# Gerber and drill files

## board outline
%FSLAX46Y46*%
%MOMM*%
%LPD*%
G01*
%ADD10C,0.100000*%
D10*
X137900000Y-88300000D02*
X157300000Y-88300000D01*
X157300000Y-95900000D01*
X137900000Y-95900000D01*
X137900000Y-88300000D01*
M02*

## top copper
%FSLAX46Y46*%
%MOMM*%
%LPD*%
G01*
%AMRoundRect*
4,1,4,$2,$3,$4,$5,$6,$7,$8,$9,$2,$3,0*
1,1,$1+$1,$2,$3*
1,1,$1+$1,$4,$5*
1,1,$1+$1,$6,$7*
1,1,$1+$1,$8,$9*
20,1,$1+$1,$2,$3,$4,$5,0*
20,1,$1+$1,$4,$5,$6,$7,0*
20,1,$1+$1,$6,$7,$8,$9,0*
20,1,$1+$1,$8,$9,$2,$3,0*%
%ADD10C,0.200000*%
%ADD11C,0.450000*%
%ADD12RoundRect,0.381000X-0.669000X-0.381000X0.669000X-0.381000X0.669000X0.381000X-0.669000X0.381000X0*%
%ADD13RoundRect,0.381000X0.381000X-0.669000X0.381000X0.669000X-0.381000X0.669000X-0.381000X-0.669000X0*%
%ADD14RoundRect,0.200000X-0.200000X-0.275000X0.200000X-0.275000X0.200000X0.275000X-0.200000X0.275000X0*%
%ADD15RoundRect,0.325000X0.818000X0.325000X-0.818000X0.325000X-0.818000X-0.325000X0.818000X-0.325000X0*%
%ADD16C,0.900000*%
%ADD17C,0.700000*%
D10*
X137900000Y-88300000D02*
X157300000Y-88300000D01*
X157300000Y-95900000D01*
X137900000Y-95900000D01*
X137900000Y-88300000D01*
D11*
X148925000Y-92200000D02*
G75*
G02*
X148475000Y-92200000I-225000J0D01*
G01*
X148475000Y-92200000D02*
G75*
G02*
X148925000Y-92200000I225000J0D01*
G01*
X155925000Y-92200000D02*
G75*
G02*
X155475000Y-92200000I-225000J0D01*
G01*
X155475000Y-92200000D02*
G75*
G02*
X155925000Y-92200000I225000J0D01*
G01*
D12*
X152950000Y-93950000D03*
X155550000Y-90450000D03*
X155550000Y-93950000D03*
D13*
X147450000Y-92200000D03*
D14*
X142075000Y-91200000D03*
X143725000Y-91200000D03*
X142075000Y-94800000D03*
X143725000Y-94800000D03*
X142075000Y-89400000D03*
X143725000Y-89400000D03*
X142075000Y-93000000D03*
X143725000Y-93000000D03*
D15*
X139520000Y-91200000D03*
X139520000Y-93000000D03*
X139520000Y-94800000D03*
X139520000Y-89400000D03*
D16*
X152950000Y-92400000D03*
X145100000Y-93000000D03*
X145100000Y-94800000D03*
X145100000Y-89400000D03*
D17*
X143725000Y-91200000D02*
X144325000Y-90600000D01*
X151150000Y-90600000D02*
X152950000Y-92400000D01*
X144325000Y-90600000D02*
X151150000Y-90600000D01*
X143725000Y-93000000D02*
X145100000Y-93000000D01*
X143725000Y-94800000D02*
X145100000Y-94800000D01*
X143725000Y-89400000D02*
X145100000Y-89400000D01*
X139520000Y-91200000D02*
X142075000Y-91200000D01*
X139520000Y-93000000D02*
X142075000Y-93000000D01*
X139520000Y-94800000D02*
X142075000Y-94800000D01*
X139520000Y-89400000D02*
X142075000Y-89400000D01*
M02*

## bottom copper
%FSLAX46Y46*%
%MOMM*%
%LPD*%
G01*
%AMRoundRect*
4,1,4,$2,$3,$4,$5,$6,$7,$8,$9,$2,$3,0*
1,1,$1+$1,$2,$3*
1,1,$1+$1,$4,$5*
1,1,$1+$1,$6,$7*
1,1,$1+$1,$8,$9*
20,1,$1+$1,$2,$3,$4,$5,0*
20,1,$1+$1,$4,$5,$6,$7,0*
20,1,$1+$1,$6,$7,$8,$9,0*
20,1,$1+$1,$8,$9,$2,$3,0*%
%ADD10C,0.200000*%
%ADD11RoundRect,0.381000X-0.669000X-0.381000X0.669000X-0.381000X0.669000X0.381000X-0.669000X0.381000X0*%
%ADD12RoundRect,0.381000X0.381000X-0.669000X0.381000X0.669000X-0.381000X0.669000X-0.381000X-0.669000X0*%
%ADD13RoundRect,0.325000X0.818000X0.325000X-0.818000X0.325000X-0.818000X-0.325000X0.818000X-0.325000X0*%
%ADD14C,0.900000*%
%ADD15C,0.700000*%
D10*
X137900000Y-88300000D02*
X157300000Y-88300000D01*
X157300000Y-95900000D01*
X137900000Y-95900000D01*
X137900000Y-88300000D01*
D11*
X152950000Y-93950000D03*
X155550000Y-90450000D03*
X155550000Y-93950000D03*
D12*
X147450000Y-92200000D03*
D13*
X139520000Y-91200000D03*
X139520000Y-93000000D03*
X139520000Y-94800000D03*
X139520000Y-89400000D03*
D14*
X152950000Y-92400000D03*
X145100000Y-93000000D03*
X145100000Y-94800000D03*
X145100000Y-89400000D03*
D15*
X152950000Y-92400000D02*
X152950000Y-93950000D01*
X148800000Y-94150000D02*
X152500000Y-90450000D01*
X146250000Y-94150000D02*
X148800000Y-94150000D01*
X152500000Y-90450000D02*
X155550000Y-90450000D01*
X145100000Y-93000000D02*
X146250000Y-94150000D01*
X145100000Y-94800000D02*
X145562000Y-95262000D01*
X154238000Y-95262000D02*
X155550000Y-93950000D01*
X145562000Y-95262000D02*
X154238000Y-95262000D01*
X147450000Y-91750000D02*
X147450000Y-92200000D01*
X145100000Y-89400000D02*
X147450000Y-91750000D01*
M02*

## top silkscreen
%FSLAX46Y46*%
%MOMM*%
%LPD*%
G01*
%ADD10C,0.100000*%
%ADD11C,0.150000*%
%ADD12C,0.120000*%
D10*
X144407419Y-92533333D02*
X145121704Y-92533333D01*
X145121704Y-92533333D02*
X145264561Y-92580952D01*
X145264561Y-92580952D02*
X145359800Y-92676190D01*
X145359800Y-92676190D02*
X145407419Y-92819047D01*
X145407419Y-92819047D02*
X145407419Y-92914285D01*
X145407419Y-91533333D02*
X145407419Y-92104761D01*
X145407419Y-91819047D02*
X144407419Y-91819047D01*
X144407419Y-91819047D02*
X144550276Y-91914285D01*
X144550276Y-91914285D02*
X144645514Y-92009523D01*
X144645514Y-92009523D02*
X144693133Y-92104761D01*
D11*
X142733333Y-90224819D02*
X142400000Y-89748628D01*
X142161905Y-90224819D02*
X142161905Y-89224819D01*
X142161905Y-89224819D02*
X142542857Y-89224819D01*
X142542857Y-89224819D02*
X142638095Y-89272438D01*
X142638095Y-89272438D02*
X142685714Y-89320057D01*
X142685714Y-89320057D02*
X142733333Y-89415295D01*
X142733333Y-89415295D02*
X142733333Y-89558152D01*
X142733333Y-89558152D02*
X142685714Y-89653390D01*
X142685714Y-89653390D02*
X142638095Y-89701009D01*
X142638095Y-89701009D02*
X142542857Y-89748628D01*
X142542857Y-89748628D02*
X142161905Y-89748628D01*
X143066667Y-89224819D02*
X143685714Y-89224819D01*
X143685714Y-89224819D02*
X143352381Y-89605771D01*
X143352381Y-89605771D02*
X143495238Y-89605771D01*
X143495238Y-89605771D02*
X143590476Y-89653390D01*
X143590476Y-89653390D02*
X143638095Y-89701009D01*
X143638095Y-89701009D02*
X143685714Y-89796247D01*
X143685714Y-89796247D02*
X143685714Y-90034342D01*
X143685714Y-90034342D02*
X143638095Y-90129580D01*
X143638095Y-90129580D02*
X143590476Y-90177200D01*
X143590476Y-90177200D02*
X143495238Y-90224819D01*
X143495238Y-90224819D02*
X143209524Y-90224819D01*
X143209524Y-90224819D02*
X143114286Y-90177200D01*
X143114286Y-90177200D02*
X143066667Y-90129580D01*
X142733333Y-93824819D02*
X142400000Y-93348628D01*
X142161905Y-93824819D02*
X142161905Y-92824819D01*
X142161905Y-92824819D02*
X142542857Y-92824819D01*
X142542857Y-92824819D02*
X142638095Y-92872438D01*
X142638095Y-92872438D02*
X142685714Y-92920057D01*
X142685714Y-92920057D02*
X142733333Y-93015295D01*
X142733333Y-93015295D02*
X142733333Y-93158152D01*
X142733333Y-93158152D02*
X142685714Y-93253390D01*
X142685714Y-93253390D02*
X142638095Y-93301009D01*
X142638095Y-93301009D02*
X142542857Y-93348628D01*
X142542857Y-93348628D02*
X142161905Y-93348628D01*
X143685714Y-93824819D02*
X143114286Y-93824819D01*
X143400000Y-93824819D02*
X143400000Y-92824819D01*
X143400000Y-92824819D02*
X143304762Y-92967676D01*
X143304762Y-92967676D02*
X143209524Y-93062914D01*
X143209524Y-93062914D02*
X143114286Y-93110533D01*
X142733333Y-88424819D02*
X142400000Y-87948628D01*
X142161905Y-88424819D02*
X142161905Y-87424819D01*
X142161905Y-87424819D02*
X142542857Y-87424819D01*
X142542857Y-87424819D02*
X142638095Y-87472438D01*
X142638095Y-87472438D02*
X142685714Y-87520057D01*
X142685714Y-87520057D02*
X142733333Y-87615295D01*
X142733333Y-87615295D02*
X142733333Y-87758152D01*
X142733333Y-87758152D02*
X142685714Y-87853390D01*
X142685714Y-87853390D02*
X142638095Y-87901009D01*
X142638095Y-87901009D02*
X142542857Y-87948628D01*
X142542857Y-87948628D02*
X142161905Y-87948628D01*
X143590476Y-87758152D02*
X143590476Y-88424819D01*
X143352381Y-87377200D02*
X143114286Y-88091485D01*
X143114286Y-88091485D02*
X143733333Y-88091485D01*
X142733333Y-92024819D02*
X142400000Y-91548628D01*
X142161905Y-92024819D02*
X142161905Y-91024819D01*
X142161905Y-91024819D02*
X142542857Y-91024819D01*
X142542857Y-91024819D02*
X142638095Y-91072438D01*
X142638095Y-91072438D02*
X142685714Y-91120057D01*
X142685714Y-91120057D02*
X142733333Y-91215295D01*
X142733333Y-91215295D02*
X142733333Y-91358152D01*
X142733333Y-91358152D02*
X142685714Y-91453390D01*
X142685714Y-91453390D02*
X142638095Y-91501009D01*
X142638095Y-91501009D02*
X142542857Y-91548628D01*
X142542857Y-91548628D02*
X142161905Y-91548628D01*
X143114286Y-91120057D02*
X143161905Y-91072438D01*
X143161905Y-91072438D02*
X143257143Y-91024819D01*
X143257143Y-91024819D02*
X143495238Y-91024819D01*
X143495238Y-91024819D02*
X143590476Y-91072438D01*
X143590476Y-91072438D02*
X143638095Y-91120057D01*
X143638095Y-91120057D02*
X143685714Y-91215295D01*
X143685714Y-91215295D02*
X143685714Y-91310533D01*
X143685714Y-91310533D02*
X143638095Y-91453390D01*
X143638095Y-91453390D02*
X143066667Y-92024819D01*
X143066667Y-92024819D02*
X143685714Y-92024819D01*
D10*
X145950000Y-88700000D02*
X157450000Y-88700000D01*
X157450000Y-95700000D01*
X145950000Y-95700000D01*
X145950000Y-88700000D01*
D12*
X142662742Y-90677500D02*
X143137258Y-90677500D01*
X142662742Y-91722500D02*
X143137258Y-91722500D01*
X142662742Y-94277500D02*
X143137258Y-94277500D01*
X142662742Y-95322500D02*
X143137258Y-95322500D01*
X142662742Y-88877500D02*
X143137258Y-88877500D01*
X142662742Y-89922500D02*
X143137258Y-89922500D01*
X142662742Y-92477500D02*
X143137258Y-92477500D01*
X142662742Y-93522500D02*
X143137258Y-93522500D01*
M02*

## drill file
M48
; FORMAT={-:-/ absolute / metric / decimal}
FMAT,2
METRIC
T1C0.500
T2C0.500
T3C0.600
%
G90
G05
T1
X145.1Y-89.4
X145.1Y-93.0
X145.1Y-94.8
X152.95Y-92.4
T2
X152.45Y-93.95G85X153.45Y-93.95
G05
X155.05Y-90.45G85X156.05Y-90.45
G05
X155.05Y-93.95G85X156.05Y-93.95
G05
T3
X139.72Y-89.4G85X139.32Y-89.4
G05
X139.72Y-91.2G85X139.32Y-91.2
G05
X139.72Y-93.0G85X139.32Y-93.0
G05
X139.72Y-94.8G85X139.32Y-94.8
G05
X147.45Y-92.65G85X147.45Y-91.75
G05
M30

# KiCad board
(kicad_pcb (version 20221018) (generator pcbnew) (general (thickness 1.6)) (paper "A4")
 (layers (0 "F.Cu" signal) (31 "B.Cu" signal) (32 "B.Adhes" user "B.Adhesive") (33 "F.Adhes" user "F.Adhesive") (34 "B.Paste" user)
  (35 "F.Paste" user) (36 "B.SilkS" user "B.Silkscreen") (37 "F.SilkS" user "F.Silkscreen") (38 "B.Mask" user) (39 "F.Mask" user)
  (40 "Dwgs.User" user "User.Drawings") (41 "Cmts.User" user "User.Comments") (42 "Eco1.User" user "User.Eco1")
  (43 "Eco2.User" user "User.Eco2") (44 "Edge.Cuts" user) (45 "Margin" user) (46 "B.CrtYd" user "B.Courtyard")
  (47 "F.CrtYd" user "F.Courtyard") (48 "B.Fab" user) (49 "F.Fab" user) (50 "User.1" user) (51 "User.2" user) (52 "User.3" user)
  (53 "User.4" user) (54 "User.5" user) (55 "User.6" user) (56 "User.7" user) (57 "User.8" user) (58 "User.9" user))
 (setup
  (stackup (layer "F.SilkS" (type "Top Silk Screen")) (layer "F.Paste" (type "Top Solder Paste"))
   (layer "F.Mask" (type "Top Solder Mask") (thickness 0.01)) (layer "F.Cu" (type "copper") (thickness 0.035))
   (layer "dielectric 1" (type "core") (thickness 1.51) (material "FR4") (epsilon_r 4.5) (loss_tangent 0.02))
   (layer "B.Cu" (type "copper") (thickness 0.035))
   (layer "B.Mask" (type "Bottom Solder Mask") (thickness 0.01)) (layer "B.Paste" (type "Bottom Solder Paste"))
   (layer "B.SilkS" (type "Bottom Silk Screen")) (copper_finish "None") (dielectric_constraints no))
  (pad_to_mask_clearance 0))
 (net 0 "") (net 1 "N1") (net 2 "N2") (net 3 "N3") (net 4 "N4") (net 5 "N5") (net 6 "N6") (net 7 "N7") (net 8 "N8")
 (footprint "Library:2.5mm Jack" (layer "F.Cu") (at 157.45 92.2 90)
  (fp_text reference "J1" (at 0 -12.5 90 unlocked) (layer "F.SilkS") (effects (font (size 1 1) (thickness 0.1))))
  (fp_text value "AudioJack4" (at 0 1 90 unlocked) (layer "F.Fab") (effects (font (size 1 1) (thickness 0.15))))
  (fp_circle (center 0 -8.75) (end 0.4 -8.75) (stroke (width 0.1) (type solid)) (fill solid) (layer "F.Cu"))
  (fp_circle (center 0 -1.75) (end 0.4 -1.75) (stroke (width 0.1) (type solid)) (fill solid) (layer "F.Cu"))
  (fp_rect (start -3.5 -11.5) (end 3.5 0) (stroke (width 0.1) (type default)) (fill none) (layer "F.SilkS"))
  (pad "R1" thru_hole roundrect (at -1.75 -4.5) (size 2.1 1.524) (drill oval 1.5 0.5) (layers "*.Cu" "*.Mask") (roundrect_rratio 0.25)
   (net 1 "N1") (thermal_bridge_angle 45))
  (pad "R2" thru_hole roundrect (at 1.75 -1.9) (size 2.1 1.524) (drill oval 1.5 0.5) (layers "*.Cu" "*.Mask") (roundrect_rratio 0.25)
   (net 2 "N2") (thermal_bridge_angle 45))
  (pad "S" thru_hole roundrect (at -1.75 -1.9) (size 2.1 1.524) (drill oval 1.5 0.5) (layers "*.Cu" "*.Mask") (roundrect_rratio 0.25)
   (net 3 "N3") (thermal_bridge_angle 45))
  (pad "T" thru_hole roundrect (at 0 -10 90) (size 2.1 1.524) (drill oval 1.5 0.6) (layers "*.Cu" "*.Mask") (roundrect_rratio 0.25)
   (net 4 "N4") (thermal_bridge_angle 45))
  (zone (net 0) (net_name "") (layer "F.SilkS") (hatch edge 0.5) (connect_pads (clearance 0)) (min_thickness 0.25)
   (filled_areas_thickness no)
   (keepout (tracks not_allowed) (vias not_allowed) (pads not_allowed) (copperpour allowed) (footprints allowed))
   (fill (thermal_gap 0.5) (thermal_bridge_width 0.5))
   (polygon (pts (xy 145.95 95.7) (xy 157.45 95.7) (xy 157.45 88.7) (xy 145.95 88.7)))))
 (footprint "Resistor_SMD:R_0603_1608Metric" (layer "F.Cu") (at 142.9 91.2)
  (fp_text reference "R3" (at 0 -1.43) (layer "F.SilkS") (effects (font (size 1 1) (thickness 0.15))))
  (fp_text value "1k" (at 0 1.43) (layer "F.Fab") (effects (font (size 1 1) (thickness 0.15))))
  (fp_line (start -0.237258 -0.5225) (end 0.237258 -0.5225) (stroke (width 0.12) (type solid)) (layer "F.SilkS"))
  (fp_line (start -0.237258 0.5225) (end 0.237258 0.5225) (stroke (width 0.12) (type solid)) (layer "F.SilkS"))
  (pad "1" smd roundrect (at -0.825 0) (size 0.8 0.95) (layers "F.Cu" "F.Paste" "F.Mask") (roundrect_rratio 0.25) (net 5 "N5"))
  (pad "2" smd roundrect (at 0.825 0) (size 0.8 0.95) (layers "F.Cu" "F.Paste" "F.Mask") (roundrect_rratio 0.25) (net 1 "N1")))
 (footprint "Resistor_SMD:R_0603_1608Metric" (layer "F.Cu") (at 142.9 94.8)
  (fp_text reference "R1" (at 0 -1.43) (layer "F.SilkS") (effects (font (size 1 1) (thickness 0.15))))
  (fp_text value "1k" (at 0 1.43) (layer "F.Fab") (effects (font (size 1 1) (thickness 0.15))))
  (fp_line (start -0.237258 -0.5225) (end 0.237258 -0.5225) (stroke (width 0.12) (type solid)) (layer "F.SilkS"))
  (fp_line (start -0.237258 0.5225) (end 0.237258 0.5225) (stroke (width 0.12) (type solid)) (layer "F.SilkS"))
  (pad "1" smd roundrect (at -0.825 0) (size 0.8 0.95) (layers "F.Cu" "F.Paste" "F.Mask") (roundrect_rratio 0.25) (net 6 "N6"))
  (pad "2" smd roundrect (at 0.825 0) (size 0.8 0.95) (layers "F.Cu" "F.Paste" "F.Mask") (roundrect_rratio 0.25) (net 3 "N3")))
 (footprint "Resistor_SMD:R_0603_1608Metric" (layer "F.Cu") (at 142.9 89.4)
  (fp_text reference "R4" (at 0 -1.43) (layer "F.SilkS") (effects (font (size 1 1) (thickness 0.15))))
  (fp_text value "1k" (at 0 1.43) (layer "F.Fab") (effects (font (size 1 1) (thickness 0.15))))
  (fp_line (start -0.237258 -0.5225) (end 0.237258 -0.5225) (stroke (width 0.12) (type solid)) (layer "F.SilkS"))
  (fp_line (start -0.237258 0.5225) (end 0.237258 0.5225) (stroke (width 0.12) (type solid)) (layer "F.SilkS"))
  (pad "1" smd roundrect (at -0.825 0) (size 0.8 0.95) (layers "F.Cu" "F.Paste" "F.Mask") (roundrect_rratio 0.25) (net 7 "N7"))
  (pad "2" smd roundrect (at 0.825 0) (size 0.8 0.95) (layers "F.Cu" "F.Paste" "F.Mask") (roundrect_rratio 0.25) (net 4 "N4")))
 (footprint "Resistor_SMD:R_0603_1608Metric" (layer "F.Cu") (at 142.9 93)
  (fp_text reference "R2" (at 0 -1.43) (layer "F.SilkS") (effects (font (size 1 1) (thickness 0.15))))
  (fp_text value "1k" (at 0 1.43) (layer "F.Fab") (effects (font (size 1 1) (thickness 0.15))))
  (fp_line (start -0.237258 -0.5225) (end 0.237258 -0.5225) (stroke (width 0.12) (type solid)) (layer "F.SilkS"))
  (fp_line (start -0.237258 0.5225) (end 0.237258 0.5225) (stroke (width 0.12) (type solid)) (layer "F.SilkS"))
  (pad "1" smd roundrect (at -0.825 0) (size 0.8 0.95) (layers "F.Cu" "F.Paste" "F.Mask") (roundrect_rratio 0.25) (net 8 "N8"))
  (pad "2" smd roundrect (at 0.825 0) (size 0.8 0.95) (layers "F.Cu" "F.Paste" "F.Mask") (roundrect_rratio 0.25) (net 2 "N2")))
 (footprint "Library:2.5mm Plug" (layer "B.Cu") (at 139.52 95.9 180)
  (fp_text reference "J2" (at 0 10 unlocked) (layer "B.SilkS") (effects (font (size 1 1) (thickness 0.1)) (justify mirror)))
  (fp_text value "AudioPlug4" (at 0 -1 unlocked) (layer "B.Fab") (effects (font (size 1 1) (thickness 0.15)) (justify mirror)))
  (pad "R1" thru_hole roundrect (at 0 4.7 180) (size 2.286 1.3) (drill oval 1 0.6) (layers "*.Cu" "*.Mask") (roundrect_rratio 0.25)
   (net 5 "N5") (thermal_bridge_angle 45))
  (pad "R2" thru_hole roundrect (at 0 2.9 180) (size 2.286 1.3) (drill oval 1 0.6) (layers "*.Cu" "*.Mask") (roundrect_rratio 0.25)
   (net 8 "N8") (thermal_bridge_angle 45))
  (pad "S" thru_hole roundrect (at 0 1.1 180) (size 2.286 1.3) (drill oval 1 0.6) (layers "*.Cu" "*.Mask") (roundrect_rratio 0.25)
   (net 6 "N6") (thermal_bridge_angle 45))
  (pad "T" thru_hole roundrect (at 0 6.5 180) (size 2.286 1.3) (drill oval 1 0.6) (layers "*.Cu" "*.Mask") (roundrect_rratio 0.25)
   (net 7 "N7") (thermal_bridge_angle 45))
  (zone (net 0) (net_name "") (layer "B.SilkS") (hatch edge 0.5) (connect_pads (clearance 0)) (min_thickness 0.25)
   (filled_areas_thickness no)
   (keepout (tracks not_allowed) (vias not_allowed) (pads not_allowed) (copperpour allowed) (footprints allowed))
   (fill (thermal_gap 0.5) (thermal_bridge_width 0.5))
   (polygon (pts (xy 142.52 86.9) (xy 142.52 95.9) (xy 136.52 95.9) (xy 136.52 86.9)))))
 (gr_rect (start 137.9 88.3) (end 157.3 95.9) (stroke (width 0.2) (type default)) (fill none) (layer "F.Cu"))
 (gr_rect (start 137.9 88.3) (end 157.3 95.9) (stroke (width 0.2) (type default)) (fill none) (layer "B.Cu"))
 (gr_rect (start 137.9 88.3) (end 157.3 95.9) (stroke (width 0.1) (type default)) (fill none) (layer "Edge.Cuts"))
 (segment (start 143.725 91.2) (end 144.325 90.6) (width 0.7) (layer "F.Cu") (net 1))
 (segment (start 151.15 90.6) (end 152.95 92.4) (width 0.7) (layer "F.Cu") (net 1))
 (segment (start 144.325 90.6) (end 151.15 90.6) (width 0.7) (layer "F.Cu") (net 1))
 (via (at 152.95 92.4) (size 0.9) (drill 0.5) (layers "F.Cu" "B.Cu") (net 1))
 (segment (start 152.95 92.4) (end 152.95 93.95) (width 0.7) (layer "B.Cu") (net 1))
 (segment (start 143.725 93) (end 145.1 93) (width 0.7) (layer "F.Cu") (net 2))
 (via (at 145.1 93) (size 0.9) (drill 0.5) (layers "F.Cu" "B.Cu") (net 2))
 (segment (start 148.8 94.15) (end 152.5 90.45) (width 0.7) (layer "B.Cu") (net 2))
 (segment (start 146.25 94.15) (end 148.8 94.15) (width 0.7) (layer "B.Cu") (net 2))
 (segment (start 152.5 90.45) (end 155.55 90.45) (width 0.7) (layer "B.Cu") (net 2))
 (segment (start 145.1 93) (end 146.25 94.15) (width 0.7) (layer "B.Cu") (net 2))
 (segment (start 143.725 94.8) (end 145.1 94.8) (width 0.7) (layer "F.Cu") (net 3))
 (via (at 145.1 94.8) (size 0.9) (drill 0.5) (layers "F.Cu" "B.Cu") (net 3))
 (segment (start 145.1 94.8) (end 145.562 95.262) (width 0.7) (layer "B.Cu") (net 3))
 (segment (start 154.238 95.262) (end 155.55 93.95) (width 0.7) (layer "B.Cu") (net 3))
 (segment (start 145.562 95.262) (end 154.238 95.262) (width 0.7) (layer "B.Cu") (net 3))
 (segment (start 143.725 89.4) (end 145.1 89.4) (width 0.7) (layer "F.Cu") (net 4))
 (via (at 145.1 89.4) (size 0.9) (drill 0.5) (layers "F.Cu" "B.Cu") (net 4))
 (segment (start 147.45 91.75) (end 147.45 92.2) (width 0.7) (layer "B.Cu") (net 4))
 (segment (start 145.1 89.4) (end 147.45 91.75) (width 0.7) (layer "B.Cu") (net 4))
 (segment (start 139.52 91.2) (end 142.075 91.2) (width 0.7) (layer "F.Cu") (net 5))
 (segment (start 139.52 93) (end 142.075 93) (width 0.7) (layer "F.Cu") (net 8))
 (segment (start 139.52 94.8) (end 142.075 94.8) (width 0.7) (layer "F.Cu") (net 6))
 (segment (start 139.52 89.4) (end 142.075 89.4) (width 0.7) (layer "F.Cu") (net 7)))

